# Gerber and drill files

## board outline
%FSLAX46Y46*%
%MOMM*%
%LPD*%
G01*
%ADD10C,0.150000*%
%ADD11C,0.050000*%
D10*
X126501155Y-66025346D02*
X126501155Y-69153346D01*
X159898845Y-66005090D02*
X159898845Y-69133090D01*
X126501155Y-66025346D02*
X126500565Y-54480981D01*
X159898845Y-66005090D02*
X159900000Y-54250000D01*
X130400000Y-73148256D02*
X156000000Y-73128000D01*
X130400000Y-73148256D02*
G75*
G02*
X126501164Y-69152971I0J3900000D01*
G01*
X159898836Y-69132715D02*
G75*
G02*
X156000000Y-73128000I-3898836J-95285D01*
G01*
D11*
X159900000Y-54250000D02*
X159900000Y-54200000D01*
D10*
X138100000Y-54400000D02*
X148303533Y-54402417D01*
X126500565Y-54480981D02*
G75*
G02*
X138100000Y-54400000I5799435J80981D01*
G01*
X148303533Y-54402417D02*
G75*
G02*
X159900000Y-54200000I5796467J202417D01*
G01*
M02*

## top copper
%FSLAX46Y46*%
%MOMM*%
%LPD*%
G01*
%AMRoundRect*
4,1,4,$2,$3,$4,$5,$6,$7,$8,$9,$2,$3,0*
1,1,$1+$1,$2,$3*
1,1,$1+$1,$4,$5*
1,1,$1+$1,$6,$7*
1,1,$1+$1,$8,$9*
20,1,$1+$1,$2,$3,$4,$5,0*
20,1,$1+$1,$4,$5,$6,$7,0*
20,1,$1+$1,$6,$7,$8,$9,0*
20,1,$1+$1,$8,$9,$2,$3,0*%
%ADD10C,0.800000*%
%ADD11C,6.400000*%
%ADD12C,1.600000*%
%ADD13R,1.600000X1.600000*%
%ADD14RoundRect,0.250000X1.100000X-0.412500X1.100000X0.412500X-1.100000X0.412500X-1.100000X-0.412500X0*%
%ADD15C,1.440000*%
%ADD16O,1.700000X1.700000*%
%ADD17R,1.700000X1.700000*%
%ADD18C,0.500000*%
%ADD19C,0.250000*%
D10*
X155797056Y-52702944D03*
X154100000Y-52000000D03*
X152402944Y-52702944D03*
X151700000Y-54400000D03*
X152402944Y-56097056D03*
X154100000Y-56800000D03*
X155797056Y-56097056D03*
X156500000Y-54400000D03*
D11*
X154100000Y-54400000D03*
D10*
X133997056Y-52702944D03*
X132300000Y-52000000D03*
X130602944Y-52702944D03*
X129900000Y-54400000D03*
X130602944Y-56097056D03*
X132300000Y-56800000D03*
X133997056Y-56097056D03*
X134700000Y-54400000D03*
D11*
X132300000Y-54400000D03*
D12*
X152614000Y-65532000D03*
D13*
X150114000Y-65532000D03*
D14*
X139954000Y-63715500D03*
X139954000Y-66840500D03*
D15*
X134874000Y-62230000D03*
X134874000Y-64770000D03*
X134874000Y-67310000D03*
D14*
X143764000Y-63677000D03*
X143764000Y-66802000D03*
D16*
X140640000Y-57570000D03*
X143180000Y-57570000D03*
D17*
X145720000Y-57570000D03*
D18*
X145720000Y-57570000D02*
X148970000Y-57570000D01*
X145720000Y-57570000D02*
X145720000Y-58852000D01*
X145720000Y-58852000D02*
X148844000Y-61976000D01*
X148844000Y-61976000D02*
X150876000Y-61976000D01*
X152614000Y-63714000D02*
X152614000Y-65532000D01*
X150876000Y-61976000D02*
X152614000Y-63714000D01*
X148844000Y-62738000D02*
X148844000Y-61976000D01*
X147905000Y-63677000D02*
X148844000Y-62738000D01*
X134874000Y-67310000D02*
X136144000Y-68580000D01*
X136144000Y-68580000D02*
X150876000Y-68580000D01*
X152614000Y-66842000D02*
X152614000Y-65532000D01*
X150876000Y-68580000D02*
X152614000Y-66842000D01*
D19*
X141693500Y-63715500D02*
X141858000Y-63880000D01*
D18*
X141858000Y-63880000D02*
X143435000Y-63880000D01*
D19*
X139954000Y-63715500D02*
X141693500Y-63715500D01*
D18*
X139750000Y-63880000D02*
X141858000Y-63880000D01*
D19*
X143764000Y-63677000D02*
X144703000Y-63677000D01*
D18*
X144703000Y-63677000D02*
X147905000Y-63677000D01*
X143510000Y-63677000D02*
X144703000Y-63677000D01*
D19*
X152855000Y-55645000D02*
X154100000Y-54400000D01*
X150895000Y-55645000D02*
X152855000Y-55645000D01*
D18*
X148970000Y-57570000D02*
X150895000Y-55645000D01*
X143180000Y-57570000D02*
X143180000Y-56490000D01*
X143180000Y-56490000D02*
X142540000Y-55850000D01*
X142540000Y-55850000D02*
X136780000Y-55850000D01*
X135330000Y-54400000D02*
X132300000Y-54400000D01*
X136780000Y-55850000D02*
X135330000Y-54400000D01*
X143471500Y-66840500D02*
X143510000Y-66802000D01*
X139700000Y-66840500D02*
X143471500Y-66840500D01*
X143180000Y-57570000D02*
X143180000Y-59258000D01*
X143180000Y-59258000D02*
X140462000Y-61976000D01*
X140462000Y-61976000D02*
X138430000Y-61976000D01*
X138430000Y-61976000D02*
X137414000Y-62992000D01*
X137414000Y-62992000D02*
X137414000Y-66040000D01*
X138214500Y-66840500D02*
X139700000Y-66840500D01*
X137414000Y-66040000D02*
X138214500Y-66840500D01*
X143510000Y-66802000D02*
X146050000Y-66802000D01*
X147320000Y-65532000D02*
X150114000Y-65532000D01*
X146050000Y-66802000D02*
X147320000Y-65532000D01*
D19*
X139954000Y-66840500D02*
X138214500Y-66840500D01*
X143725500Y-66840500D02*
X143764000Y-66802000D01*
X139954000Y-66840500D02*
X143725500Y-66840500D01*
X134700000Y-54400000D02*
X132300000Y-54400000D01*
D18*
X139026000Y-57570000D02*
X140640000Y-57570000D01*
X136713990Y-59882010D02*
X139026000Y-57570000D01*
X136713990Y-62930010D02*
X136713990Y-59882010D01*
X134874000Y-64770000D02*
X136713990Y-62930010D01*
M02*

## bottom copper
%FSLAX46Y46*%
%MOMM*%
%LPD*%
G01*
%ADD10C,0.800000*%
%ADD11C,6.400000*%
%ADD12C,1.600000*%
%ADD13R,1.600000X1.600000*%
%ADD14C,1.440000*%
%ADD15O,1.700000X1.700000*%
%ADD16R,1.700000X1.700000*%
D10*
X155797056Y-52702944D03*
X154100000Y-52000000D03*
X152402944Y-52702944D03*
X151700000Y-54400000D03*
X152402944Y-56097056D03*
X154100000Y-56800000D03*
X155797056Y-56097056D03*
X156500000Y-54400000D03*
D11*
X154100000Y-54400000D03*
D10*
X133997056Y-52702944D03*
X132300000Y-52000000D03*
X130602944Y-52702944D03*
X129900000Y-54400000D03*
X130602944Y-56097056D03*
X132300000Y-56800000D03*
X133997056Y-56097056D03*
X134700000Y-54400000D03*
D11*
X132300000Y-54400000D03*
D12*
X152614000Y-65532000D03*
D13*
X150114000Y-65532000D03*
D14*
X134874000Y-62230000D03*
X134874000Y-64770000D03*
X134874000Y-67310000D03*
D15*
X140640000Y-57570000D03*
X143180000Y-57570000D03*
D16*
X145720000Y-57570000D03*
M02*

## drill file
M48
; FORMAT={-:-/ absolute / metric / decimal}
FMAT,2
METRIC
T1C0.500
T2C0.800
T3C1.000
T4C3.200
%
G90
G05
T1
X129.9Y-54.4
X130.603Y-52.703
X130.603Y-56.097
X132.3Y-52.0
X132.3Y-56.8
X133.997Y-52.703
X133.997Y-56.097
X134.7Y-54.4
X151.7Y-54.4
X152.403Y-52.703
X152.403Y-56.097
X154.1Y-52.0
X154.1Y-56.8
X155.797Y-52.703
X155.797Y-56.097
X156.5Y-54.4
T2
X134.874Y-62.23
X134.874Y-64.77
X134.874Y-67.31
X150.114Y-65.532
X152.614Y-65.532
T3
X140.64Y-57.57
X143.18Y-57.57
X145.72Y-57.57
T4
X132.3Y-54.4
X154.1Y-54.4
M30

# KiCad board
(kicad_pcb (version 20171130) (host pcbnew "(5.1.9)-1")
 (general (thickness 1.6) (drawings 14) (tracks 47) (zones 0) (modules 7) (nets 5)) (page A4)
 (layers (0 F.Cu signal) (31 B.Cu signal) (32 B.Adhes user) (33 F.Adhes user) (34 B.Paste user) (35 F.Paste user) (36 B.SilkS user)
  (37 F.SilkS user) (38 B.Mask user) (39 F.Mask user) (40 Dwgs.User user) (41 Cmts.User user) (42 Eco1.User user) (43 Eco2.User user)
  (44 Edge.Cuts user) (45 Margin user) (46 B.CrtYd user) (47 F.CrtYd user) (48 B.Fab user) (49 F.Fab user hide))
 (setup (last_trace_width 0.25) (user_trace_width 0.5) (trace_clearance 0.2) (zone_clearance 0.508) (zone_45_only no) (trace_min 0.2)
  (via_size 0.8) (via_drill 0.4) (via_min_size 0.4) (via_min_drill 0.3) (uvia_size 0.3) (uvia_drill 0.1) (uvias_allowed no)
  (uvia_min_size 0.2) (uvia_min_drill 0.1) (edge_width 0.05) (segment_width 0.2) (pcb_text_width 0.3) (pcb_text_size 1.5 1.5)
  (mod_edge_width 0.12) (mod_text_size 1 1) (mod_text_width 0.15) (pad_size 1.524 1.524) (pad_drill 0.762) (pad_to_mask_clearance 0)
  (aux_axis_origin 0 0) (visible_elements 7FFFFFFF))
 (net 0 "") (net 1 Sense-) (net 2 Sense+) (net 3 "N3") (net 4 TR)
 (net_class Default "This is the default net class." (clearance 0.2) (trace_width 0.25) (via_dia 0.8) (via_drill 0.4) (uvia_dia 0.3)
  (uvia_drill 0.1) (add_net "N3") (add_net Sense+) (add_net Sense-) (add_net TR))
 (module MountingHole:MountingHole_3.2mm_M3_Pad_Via (layer F.Cu) (at 154.1 54.4)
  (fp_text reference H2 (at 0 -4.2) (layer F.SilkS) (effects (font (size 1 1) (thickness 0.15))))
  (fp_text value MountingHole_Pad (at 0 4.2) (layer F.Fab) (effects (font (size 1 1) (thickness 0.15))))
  (pad 1 thru_hole circle (at 1.697056 -1.697056) (size 0.8 0.8) (drill 0.5) (layers *.Cu *.Mask) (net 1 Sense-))
  (pad 1 thru_hole circle (at 0 -2.4) (size 0.8 0.8) (drill 0.5) (layers *.Cu *.Mask) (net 1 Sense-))
  (pad 1 thru_hole circle (at -1.697056 -1.697056) (size 0.8 0.8) (drill 0.5) (layers *.Cu *.Mask) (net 1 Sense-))
  (pad 1 thru_hole circle (at -2.4 0) (size 0.8 0.8) (drill 0.5) (layers *.Cu *.Mask) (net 1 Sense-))
  (pad 1 thru_hole circle (at -1.697056 1.697056) (size 0.8 0.8) (drill 0.5) (layers *.Cu *.Mask) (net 1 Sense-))
  (pad 1 thru_hole circle (at 0 2.4) (size 0.8 0.8) (drill 0.5) (layers *.Cu *.Mask) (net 1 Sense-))
  (pad 1 thru_hole circle (at 1.697056 1.697056) (size 0.8 0.8) (drill 0.5) (layers *.Cu *.Mask) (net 1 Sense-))
  (pad 1 thru_hole circle (at 2.4 0) (size 0.8 0.8) (drill 0.5) (layers *.Cu *.Mask) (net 1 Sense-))
  (pad 1 thru_hole circle (at 0 0) (size 6.4 6.4) (drill 3.2) (layers *.Cu *.Mask) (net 1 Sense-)))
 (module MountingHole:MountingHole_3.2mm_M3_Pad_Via (layer F.Cu) (at 132.3 54.4)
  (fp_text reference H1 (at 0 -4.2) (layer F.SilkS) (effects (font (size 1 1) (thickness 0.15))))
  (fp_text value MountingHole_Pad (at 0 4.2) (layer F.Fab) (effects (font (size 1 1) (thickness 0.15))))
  (pad 1 thru_hole circle (at 1.697056 -1.697056) (size 0.8 0.8) (drill 0.5) (layers *.Cu *.Mask) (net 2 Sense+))
  (pad 1 thru_hole circle (at 0 -2.4) (size 0.8 0.8) (drill 0.5) (layers *.Cu *.Mask) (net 2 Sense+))
  (pad 1 thru_hole circle (at -1.697056 -1.697056) (size 0.8 0.8) (drill 0.5) (layers *.Cu *.Mask) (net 2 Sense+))
  (pad 1 thru_hole circle (at -2.4 0) (size 0.8 0.8) (drill 0.5) (layers *.Cu *.Mask) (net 2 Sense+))
  (pad 1 thru_hole circle (at -1.697056 1.697056) (size 0.8 0.8) (drill 0.5) (layers *.Cu *.Mask) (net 2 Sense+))
  (pad 1 thru_hole circle (at 0 2.4) (size 0.8 0.8) (drill 0.5) (layers *.Cu *.Mask) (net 2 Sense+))
  (pad 1 thru_hole circle (at 1.697056 1.697056) (size 0.8 0.8) (drill 0.5) (layers *.Cu *.Mask) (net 2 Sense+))
  (pad 1 thru_hole circle (at 2.4 0) (size 0.8 0.8) (drill 0.5) (layers *.Cu *.Mask) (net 2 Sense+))
  (pad 1 thru_hole circle (at 0 0) (size 6.4 6.4) (drill 3.2) (layers *.Cu *.Mask) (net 2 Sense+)))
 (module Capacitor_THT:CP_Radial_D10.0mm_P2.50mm (layer F.Cu) (at 150.114 65.532)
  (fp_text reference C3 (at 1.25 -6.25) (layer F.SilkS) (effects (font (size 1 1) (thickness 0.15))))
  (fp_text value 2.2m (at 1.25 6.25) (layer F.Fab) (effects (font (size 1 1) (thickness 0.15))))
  (pad 2 thru_hole circle (at 2.5 0) (size 1.6 1.6) (drill 0.8) (layers *.Cu *.Mask) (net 1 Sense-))
  (pad 1 thru_hole rect (at 0 0) (size 1.6 1.6) (drill 0.8) (layers *.Cu *.Mask) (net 2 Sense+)))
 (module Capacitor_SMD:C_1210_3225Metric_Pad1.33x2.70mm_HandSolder (layer F.Cu) (at 139.954 65.278 90)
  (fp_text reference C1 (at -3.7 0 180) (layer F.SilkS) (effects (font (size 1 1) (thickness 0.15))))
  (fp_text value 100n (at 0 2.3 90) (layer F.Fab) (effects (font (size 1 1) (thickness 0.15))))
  (pad 2 smd roundrect (at 1.5625 0 90) (size 1.325 2.7) (layers F.Cu F.Paste F.Mask) (roundrect_rratio 0.188679) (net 1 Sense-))
  (pad 1 smd roundrect (at -1.5625 0 90) (size 1.325 2.7) (layers F.Cu F.Paste F.Mask) (roundrect_rratio 0.188679) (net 2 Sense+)))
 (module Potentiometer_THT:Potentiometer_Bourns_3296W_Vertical (layer F.Cu) (at 134.874 67.31 270)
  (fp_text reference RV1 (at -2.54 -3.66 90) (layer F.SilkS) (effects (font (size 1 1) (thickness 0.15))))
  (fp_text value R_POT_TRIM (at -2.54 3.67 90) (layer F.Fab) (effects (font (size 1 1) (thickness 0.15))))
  (pad 3 thru_hole circle (at -5.08 0 270) (size 1.44 1.44) (drill 0.8) (layers *.Cu *.Mask) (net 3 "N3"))
  (pad 2 thru_hole circle (at -2.54 0 270) (size 1.44 1.44) (drill 0.8) (layers *.Cu *.Mask) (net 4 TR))
  (pad 1 thru_hole circle (at 0 0 270) (size 1.44 1.44) (drill 0.8) (layers *.Cu *.Mask) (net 1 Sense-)))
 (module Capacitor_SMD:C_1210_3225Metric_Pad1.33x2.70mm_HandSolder (layer F.Cu) (at 143.764 65.2395 90)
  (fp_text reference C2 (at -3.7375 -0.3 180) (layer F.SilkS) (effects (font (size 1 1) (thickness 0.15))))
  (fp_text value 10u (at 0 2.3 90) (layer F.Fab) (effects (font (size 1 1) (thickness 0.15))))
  (pad 2 smd roundrect (at 1.5625 0 90) (size 1.325 2.7) (layers F.Cu F.Paste F.Mask) (roundrect_rratio 0.188679) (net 1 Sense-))
  (pad 1 smd roundrect (at -1.5625 0 90) (size 1.325 2.7) (layers F.Cu F.Paste F.Mask) (roundrect_rratio 0.188679) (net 2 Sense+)))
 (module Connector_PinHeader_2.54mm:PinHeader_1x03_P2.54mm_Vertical (layer F.Cu) (at 145.72 57.57 270)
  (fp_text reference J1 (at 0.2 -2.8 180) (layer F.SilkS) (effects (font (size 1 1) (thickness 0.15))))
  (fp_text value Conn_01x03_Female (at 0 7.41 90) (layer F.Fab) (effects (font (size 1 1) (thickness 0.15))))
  (pad 3 thru_hole oval (at 0 5.08 270) (size 1.7 1.7) (drill 1) (layers *.Cu *.Mask) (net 4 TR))
  (pad 2 thru_hole oval (at 0 2.54 270) (size 1.7 1.7) (drill 1) (layers *.Cu *.Mask) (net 2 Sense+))
  (pad 1 thru_hole rect (at 0 0 270) (size 1.7 1.7) (drill 1) (layers *.Cu *.Mask) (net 1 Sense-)))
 (gr_line (start 126.501155 66.025346) (end 126.501155 69.153346) (layer Edge.Cuts) (width 0.15))
 (gr_line (start 159.898845 66.00509) (end 159.898845 69.13309) (layer Edge.Cuts) (width 0.15))
 (gr_line (start 126.501155 66.025346) (end 126.500565 54.480981) (layer Edge.Cuts) (width 0.15))
 (gr_line (start 159.898845 66.00509) (end 159.9 54.25) (layer Edge.Cuts) (width 0.15))
 (gr_line (start 130.4 73.148256) (end 156 73.128) (layer Edge.Cuts) (width 0.15))
 (gr_arc (start 130.4 69.248256) (end 130.4 73.148256) (angle 91.4) (layer Edge.Cuts) (width 0.15))
 (gr_arc (start 156 69.228) (end 156 73.128) (angle -91.4) (layer Edge.Cuts) (width 0.15))
 (gr_line (start 159.9 54.25) (end 159.9 54.2) (layer Edge.Cuts) (width 0.05))
 (gr_line (start 138.1 54.4) (end 148.303533 54.402417) (layer Edge.Cuts) (width 0.15))
 (gr_arc (start 132.3 54.4) (end 138.1 54.4) (angle -180.8) (layer Edge.Cuts) (width 0.15))
 (gr_arc (start 154.1 54.2) (end 159.9 54.2) (angle -182) (layer Edge.Cuts) (width 0.15))
 (segment (start 145.72 57.57) (end 148.97 57.57) (width 0.5) (layer F.Cu) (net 1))
 (segment (start 145.72 57.57) (end 145.72 58.852) (width 0.5) (layer F.Cu) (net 1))
 (segment (start 145.72 58.852) (end 148.844 61.976) (width 0.5) (layer F.Cu) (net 1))
 (segment (start 148.844 61.976) (end 150.876 61.976) (width 0.5) (layer F.Cu) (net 1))
 (segment (start 152.614 63.714) (end 152.614 65.532) (width 0.5) (layer F.Cu) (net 1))
 (segment (start 150.876 61.976) (end 152.614 63.714) (width 0.5) (layer F.Cu) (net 1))
 (segment (start 148.844 62.738) (end 148.844 61.976) (width 0.5) (layer F.Cu) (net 1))
 (segment (start 147.905 63.677) (end 148.844 62.738) (width 0.5) (layer F.Cu) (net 1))
 (segment (start 134.874 67.31) (end 136.144 68.58) (width 0.5) (layer F.Cu) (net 1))
 (segment (start 136.144 68.58) (end 150.876 68.58) (width 0.5) (layer F.Cu) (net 1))
 (segment (start 152.614 66.842) (end 152.614 65.532) (width 0.5) (layer F.Cu) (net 1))
 (segment (start 150.876 68.58) (end 152.614 66.842) (width 0.5) (layer F.Cu) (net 1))
 (segment (start 141.6935 63.7155) (end 141.858 63.88) (width 0.25) (layer F.Cu) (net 1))
 (segment (start 141.858 63.88) (end 143.435 63.88) (width 0.5) (layer F.Cu) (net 1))
 (segment (start 139.954 63.7155) (end 141.6935 63.7155) (width 0.25) (layer F.Cu) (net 1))
 (segment (start 139.75 63.88) (end 141.858 63.88) (width 0.5) (layer F.Cu) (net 1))
 (segment (start 143.764 63.677) (end 144.703 63.677) (width 0.25) (layer F.Cu) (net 1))
 (segment (start 144.703 63.677) (end 147.905 63.677) (width 0.5) (layer F.Cu) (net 1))
 (segment (start 143.51 63.677) (end 144.703 63.677) (width 0.5) (layer F.Cu) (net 1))
 (segment (start 152.855 55.645) (end 154.1 54.4) (width 0.25) (layer F.Cu) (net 1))
 (segment (start 150.895 55.645) (end 152.855 55.645) (width 0.25) (layer F.Cu) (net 1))
 (segment (start 148.97 57.57) (end 150.895 55.645) (width 0.5) (layer F.Cu) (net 1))
 (segment (start 143.18 57.57) (end 143.18 56.49) (width 0.5) (layer F.Cu) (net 2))
 (segment (start 143.18 56.49) (end 142.54 55.85) (width 0.5) (layer F.Cu) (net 2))
 (segment (start 142.54 55.85) (end 136.78 55.85) (width 0.5) (layer F.Cu) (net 2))
 (segment (start 135.33 54.4) (end 132.3 54.4) (width 0.5) (layer F.Cu) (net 2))
 (segment (start 136.78 55.85) (end 135.33 54.4) (width 0.5) (layer F.Cu) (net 2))
 (segment (start 143.4715 66.8405) (end 143.51 66.802) (width 0.5) (layer F.Cu) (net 2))
 (segment (start 139.7 66.8405) (end 143.4715 66.8405) (width 0.5) (layer F.Cu) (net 2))
 (segment (start 143.18 57.57) (end 143.18 59.258) (width 0.5) (layer F.Cu) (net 2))
 (segment (start 143.18 59.258) (end 140.462 61.976) (width 0.5) (layer F.Cu) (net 2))
 (segment (start 140.462 61.976) (end 138.43 61.976) (width 0.5) (layer F.Cu) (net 2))
 (segment (start 138.43 61.976) (end 137.414 62.992) (width 0.5) (layer F.Cu) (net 2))
 (segment (start 137.414 62.992) (end 137.414 66.04) (width 0.5) (layer F.Cu) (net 2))
 (segment (start 138.2145 66.8405) (end 139.7 66.8405) (width 0.5) (layer F.Cu) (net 2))
 (segment (start 137.414 66.04) (end 138.2145 66.8405) (width 0.5) (layer F.Cu) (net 2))
 (segment (start 143.51 66.802) (end 146.05 66.802) (width 0.5) (layer F.Cu) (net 2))
 (segment (start 147.32 65.532) (end 150.114 65.532) (width 0.5) (layer F.Cu) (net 2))
 (segment (start 146.05 66.802) (end 147.32 65.532) (width 0.5) (layer F.Cu) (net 2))
 (segment (start 139.954 66.8405) (end 138.2145 66.8405) (width 0.25) (layer F.Cu) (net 2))
 (segment (start 143.7255 66.8405) (end 143.764 66.802) (width 0.25) (layer F.Cu) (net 2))
 (segment (start 139.954 66.8405) (end 143.7255 66.8405) (width 0.25) (layer F.Cu) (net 2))
 (segment (start 134.7 54.4) (end 132.3 54.4) (width 0.25) (layer F.Cu) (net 2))
 (segment (start 139.026 57.57) (end 140.64 57.57) (width 0.5) (layer F.Cu) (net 4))
 (segment (start 136.71399 59.88201) (end 139.026 57.57) (width 0.5) (layer F.Cu) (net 4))
 (segment (start 136.71399 62.93001) (end 136.71399 59.88201) (width 0.5) (layer F.Cu) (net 4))
 (segment (start 134.874 64.77) (end 136.71399 62.93001) (width 0.5) (layer F.Cu) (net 4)))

